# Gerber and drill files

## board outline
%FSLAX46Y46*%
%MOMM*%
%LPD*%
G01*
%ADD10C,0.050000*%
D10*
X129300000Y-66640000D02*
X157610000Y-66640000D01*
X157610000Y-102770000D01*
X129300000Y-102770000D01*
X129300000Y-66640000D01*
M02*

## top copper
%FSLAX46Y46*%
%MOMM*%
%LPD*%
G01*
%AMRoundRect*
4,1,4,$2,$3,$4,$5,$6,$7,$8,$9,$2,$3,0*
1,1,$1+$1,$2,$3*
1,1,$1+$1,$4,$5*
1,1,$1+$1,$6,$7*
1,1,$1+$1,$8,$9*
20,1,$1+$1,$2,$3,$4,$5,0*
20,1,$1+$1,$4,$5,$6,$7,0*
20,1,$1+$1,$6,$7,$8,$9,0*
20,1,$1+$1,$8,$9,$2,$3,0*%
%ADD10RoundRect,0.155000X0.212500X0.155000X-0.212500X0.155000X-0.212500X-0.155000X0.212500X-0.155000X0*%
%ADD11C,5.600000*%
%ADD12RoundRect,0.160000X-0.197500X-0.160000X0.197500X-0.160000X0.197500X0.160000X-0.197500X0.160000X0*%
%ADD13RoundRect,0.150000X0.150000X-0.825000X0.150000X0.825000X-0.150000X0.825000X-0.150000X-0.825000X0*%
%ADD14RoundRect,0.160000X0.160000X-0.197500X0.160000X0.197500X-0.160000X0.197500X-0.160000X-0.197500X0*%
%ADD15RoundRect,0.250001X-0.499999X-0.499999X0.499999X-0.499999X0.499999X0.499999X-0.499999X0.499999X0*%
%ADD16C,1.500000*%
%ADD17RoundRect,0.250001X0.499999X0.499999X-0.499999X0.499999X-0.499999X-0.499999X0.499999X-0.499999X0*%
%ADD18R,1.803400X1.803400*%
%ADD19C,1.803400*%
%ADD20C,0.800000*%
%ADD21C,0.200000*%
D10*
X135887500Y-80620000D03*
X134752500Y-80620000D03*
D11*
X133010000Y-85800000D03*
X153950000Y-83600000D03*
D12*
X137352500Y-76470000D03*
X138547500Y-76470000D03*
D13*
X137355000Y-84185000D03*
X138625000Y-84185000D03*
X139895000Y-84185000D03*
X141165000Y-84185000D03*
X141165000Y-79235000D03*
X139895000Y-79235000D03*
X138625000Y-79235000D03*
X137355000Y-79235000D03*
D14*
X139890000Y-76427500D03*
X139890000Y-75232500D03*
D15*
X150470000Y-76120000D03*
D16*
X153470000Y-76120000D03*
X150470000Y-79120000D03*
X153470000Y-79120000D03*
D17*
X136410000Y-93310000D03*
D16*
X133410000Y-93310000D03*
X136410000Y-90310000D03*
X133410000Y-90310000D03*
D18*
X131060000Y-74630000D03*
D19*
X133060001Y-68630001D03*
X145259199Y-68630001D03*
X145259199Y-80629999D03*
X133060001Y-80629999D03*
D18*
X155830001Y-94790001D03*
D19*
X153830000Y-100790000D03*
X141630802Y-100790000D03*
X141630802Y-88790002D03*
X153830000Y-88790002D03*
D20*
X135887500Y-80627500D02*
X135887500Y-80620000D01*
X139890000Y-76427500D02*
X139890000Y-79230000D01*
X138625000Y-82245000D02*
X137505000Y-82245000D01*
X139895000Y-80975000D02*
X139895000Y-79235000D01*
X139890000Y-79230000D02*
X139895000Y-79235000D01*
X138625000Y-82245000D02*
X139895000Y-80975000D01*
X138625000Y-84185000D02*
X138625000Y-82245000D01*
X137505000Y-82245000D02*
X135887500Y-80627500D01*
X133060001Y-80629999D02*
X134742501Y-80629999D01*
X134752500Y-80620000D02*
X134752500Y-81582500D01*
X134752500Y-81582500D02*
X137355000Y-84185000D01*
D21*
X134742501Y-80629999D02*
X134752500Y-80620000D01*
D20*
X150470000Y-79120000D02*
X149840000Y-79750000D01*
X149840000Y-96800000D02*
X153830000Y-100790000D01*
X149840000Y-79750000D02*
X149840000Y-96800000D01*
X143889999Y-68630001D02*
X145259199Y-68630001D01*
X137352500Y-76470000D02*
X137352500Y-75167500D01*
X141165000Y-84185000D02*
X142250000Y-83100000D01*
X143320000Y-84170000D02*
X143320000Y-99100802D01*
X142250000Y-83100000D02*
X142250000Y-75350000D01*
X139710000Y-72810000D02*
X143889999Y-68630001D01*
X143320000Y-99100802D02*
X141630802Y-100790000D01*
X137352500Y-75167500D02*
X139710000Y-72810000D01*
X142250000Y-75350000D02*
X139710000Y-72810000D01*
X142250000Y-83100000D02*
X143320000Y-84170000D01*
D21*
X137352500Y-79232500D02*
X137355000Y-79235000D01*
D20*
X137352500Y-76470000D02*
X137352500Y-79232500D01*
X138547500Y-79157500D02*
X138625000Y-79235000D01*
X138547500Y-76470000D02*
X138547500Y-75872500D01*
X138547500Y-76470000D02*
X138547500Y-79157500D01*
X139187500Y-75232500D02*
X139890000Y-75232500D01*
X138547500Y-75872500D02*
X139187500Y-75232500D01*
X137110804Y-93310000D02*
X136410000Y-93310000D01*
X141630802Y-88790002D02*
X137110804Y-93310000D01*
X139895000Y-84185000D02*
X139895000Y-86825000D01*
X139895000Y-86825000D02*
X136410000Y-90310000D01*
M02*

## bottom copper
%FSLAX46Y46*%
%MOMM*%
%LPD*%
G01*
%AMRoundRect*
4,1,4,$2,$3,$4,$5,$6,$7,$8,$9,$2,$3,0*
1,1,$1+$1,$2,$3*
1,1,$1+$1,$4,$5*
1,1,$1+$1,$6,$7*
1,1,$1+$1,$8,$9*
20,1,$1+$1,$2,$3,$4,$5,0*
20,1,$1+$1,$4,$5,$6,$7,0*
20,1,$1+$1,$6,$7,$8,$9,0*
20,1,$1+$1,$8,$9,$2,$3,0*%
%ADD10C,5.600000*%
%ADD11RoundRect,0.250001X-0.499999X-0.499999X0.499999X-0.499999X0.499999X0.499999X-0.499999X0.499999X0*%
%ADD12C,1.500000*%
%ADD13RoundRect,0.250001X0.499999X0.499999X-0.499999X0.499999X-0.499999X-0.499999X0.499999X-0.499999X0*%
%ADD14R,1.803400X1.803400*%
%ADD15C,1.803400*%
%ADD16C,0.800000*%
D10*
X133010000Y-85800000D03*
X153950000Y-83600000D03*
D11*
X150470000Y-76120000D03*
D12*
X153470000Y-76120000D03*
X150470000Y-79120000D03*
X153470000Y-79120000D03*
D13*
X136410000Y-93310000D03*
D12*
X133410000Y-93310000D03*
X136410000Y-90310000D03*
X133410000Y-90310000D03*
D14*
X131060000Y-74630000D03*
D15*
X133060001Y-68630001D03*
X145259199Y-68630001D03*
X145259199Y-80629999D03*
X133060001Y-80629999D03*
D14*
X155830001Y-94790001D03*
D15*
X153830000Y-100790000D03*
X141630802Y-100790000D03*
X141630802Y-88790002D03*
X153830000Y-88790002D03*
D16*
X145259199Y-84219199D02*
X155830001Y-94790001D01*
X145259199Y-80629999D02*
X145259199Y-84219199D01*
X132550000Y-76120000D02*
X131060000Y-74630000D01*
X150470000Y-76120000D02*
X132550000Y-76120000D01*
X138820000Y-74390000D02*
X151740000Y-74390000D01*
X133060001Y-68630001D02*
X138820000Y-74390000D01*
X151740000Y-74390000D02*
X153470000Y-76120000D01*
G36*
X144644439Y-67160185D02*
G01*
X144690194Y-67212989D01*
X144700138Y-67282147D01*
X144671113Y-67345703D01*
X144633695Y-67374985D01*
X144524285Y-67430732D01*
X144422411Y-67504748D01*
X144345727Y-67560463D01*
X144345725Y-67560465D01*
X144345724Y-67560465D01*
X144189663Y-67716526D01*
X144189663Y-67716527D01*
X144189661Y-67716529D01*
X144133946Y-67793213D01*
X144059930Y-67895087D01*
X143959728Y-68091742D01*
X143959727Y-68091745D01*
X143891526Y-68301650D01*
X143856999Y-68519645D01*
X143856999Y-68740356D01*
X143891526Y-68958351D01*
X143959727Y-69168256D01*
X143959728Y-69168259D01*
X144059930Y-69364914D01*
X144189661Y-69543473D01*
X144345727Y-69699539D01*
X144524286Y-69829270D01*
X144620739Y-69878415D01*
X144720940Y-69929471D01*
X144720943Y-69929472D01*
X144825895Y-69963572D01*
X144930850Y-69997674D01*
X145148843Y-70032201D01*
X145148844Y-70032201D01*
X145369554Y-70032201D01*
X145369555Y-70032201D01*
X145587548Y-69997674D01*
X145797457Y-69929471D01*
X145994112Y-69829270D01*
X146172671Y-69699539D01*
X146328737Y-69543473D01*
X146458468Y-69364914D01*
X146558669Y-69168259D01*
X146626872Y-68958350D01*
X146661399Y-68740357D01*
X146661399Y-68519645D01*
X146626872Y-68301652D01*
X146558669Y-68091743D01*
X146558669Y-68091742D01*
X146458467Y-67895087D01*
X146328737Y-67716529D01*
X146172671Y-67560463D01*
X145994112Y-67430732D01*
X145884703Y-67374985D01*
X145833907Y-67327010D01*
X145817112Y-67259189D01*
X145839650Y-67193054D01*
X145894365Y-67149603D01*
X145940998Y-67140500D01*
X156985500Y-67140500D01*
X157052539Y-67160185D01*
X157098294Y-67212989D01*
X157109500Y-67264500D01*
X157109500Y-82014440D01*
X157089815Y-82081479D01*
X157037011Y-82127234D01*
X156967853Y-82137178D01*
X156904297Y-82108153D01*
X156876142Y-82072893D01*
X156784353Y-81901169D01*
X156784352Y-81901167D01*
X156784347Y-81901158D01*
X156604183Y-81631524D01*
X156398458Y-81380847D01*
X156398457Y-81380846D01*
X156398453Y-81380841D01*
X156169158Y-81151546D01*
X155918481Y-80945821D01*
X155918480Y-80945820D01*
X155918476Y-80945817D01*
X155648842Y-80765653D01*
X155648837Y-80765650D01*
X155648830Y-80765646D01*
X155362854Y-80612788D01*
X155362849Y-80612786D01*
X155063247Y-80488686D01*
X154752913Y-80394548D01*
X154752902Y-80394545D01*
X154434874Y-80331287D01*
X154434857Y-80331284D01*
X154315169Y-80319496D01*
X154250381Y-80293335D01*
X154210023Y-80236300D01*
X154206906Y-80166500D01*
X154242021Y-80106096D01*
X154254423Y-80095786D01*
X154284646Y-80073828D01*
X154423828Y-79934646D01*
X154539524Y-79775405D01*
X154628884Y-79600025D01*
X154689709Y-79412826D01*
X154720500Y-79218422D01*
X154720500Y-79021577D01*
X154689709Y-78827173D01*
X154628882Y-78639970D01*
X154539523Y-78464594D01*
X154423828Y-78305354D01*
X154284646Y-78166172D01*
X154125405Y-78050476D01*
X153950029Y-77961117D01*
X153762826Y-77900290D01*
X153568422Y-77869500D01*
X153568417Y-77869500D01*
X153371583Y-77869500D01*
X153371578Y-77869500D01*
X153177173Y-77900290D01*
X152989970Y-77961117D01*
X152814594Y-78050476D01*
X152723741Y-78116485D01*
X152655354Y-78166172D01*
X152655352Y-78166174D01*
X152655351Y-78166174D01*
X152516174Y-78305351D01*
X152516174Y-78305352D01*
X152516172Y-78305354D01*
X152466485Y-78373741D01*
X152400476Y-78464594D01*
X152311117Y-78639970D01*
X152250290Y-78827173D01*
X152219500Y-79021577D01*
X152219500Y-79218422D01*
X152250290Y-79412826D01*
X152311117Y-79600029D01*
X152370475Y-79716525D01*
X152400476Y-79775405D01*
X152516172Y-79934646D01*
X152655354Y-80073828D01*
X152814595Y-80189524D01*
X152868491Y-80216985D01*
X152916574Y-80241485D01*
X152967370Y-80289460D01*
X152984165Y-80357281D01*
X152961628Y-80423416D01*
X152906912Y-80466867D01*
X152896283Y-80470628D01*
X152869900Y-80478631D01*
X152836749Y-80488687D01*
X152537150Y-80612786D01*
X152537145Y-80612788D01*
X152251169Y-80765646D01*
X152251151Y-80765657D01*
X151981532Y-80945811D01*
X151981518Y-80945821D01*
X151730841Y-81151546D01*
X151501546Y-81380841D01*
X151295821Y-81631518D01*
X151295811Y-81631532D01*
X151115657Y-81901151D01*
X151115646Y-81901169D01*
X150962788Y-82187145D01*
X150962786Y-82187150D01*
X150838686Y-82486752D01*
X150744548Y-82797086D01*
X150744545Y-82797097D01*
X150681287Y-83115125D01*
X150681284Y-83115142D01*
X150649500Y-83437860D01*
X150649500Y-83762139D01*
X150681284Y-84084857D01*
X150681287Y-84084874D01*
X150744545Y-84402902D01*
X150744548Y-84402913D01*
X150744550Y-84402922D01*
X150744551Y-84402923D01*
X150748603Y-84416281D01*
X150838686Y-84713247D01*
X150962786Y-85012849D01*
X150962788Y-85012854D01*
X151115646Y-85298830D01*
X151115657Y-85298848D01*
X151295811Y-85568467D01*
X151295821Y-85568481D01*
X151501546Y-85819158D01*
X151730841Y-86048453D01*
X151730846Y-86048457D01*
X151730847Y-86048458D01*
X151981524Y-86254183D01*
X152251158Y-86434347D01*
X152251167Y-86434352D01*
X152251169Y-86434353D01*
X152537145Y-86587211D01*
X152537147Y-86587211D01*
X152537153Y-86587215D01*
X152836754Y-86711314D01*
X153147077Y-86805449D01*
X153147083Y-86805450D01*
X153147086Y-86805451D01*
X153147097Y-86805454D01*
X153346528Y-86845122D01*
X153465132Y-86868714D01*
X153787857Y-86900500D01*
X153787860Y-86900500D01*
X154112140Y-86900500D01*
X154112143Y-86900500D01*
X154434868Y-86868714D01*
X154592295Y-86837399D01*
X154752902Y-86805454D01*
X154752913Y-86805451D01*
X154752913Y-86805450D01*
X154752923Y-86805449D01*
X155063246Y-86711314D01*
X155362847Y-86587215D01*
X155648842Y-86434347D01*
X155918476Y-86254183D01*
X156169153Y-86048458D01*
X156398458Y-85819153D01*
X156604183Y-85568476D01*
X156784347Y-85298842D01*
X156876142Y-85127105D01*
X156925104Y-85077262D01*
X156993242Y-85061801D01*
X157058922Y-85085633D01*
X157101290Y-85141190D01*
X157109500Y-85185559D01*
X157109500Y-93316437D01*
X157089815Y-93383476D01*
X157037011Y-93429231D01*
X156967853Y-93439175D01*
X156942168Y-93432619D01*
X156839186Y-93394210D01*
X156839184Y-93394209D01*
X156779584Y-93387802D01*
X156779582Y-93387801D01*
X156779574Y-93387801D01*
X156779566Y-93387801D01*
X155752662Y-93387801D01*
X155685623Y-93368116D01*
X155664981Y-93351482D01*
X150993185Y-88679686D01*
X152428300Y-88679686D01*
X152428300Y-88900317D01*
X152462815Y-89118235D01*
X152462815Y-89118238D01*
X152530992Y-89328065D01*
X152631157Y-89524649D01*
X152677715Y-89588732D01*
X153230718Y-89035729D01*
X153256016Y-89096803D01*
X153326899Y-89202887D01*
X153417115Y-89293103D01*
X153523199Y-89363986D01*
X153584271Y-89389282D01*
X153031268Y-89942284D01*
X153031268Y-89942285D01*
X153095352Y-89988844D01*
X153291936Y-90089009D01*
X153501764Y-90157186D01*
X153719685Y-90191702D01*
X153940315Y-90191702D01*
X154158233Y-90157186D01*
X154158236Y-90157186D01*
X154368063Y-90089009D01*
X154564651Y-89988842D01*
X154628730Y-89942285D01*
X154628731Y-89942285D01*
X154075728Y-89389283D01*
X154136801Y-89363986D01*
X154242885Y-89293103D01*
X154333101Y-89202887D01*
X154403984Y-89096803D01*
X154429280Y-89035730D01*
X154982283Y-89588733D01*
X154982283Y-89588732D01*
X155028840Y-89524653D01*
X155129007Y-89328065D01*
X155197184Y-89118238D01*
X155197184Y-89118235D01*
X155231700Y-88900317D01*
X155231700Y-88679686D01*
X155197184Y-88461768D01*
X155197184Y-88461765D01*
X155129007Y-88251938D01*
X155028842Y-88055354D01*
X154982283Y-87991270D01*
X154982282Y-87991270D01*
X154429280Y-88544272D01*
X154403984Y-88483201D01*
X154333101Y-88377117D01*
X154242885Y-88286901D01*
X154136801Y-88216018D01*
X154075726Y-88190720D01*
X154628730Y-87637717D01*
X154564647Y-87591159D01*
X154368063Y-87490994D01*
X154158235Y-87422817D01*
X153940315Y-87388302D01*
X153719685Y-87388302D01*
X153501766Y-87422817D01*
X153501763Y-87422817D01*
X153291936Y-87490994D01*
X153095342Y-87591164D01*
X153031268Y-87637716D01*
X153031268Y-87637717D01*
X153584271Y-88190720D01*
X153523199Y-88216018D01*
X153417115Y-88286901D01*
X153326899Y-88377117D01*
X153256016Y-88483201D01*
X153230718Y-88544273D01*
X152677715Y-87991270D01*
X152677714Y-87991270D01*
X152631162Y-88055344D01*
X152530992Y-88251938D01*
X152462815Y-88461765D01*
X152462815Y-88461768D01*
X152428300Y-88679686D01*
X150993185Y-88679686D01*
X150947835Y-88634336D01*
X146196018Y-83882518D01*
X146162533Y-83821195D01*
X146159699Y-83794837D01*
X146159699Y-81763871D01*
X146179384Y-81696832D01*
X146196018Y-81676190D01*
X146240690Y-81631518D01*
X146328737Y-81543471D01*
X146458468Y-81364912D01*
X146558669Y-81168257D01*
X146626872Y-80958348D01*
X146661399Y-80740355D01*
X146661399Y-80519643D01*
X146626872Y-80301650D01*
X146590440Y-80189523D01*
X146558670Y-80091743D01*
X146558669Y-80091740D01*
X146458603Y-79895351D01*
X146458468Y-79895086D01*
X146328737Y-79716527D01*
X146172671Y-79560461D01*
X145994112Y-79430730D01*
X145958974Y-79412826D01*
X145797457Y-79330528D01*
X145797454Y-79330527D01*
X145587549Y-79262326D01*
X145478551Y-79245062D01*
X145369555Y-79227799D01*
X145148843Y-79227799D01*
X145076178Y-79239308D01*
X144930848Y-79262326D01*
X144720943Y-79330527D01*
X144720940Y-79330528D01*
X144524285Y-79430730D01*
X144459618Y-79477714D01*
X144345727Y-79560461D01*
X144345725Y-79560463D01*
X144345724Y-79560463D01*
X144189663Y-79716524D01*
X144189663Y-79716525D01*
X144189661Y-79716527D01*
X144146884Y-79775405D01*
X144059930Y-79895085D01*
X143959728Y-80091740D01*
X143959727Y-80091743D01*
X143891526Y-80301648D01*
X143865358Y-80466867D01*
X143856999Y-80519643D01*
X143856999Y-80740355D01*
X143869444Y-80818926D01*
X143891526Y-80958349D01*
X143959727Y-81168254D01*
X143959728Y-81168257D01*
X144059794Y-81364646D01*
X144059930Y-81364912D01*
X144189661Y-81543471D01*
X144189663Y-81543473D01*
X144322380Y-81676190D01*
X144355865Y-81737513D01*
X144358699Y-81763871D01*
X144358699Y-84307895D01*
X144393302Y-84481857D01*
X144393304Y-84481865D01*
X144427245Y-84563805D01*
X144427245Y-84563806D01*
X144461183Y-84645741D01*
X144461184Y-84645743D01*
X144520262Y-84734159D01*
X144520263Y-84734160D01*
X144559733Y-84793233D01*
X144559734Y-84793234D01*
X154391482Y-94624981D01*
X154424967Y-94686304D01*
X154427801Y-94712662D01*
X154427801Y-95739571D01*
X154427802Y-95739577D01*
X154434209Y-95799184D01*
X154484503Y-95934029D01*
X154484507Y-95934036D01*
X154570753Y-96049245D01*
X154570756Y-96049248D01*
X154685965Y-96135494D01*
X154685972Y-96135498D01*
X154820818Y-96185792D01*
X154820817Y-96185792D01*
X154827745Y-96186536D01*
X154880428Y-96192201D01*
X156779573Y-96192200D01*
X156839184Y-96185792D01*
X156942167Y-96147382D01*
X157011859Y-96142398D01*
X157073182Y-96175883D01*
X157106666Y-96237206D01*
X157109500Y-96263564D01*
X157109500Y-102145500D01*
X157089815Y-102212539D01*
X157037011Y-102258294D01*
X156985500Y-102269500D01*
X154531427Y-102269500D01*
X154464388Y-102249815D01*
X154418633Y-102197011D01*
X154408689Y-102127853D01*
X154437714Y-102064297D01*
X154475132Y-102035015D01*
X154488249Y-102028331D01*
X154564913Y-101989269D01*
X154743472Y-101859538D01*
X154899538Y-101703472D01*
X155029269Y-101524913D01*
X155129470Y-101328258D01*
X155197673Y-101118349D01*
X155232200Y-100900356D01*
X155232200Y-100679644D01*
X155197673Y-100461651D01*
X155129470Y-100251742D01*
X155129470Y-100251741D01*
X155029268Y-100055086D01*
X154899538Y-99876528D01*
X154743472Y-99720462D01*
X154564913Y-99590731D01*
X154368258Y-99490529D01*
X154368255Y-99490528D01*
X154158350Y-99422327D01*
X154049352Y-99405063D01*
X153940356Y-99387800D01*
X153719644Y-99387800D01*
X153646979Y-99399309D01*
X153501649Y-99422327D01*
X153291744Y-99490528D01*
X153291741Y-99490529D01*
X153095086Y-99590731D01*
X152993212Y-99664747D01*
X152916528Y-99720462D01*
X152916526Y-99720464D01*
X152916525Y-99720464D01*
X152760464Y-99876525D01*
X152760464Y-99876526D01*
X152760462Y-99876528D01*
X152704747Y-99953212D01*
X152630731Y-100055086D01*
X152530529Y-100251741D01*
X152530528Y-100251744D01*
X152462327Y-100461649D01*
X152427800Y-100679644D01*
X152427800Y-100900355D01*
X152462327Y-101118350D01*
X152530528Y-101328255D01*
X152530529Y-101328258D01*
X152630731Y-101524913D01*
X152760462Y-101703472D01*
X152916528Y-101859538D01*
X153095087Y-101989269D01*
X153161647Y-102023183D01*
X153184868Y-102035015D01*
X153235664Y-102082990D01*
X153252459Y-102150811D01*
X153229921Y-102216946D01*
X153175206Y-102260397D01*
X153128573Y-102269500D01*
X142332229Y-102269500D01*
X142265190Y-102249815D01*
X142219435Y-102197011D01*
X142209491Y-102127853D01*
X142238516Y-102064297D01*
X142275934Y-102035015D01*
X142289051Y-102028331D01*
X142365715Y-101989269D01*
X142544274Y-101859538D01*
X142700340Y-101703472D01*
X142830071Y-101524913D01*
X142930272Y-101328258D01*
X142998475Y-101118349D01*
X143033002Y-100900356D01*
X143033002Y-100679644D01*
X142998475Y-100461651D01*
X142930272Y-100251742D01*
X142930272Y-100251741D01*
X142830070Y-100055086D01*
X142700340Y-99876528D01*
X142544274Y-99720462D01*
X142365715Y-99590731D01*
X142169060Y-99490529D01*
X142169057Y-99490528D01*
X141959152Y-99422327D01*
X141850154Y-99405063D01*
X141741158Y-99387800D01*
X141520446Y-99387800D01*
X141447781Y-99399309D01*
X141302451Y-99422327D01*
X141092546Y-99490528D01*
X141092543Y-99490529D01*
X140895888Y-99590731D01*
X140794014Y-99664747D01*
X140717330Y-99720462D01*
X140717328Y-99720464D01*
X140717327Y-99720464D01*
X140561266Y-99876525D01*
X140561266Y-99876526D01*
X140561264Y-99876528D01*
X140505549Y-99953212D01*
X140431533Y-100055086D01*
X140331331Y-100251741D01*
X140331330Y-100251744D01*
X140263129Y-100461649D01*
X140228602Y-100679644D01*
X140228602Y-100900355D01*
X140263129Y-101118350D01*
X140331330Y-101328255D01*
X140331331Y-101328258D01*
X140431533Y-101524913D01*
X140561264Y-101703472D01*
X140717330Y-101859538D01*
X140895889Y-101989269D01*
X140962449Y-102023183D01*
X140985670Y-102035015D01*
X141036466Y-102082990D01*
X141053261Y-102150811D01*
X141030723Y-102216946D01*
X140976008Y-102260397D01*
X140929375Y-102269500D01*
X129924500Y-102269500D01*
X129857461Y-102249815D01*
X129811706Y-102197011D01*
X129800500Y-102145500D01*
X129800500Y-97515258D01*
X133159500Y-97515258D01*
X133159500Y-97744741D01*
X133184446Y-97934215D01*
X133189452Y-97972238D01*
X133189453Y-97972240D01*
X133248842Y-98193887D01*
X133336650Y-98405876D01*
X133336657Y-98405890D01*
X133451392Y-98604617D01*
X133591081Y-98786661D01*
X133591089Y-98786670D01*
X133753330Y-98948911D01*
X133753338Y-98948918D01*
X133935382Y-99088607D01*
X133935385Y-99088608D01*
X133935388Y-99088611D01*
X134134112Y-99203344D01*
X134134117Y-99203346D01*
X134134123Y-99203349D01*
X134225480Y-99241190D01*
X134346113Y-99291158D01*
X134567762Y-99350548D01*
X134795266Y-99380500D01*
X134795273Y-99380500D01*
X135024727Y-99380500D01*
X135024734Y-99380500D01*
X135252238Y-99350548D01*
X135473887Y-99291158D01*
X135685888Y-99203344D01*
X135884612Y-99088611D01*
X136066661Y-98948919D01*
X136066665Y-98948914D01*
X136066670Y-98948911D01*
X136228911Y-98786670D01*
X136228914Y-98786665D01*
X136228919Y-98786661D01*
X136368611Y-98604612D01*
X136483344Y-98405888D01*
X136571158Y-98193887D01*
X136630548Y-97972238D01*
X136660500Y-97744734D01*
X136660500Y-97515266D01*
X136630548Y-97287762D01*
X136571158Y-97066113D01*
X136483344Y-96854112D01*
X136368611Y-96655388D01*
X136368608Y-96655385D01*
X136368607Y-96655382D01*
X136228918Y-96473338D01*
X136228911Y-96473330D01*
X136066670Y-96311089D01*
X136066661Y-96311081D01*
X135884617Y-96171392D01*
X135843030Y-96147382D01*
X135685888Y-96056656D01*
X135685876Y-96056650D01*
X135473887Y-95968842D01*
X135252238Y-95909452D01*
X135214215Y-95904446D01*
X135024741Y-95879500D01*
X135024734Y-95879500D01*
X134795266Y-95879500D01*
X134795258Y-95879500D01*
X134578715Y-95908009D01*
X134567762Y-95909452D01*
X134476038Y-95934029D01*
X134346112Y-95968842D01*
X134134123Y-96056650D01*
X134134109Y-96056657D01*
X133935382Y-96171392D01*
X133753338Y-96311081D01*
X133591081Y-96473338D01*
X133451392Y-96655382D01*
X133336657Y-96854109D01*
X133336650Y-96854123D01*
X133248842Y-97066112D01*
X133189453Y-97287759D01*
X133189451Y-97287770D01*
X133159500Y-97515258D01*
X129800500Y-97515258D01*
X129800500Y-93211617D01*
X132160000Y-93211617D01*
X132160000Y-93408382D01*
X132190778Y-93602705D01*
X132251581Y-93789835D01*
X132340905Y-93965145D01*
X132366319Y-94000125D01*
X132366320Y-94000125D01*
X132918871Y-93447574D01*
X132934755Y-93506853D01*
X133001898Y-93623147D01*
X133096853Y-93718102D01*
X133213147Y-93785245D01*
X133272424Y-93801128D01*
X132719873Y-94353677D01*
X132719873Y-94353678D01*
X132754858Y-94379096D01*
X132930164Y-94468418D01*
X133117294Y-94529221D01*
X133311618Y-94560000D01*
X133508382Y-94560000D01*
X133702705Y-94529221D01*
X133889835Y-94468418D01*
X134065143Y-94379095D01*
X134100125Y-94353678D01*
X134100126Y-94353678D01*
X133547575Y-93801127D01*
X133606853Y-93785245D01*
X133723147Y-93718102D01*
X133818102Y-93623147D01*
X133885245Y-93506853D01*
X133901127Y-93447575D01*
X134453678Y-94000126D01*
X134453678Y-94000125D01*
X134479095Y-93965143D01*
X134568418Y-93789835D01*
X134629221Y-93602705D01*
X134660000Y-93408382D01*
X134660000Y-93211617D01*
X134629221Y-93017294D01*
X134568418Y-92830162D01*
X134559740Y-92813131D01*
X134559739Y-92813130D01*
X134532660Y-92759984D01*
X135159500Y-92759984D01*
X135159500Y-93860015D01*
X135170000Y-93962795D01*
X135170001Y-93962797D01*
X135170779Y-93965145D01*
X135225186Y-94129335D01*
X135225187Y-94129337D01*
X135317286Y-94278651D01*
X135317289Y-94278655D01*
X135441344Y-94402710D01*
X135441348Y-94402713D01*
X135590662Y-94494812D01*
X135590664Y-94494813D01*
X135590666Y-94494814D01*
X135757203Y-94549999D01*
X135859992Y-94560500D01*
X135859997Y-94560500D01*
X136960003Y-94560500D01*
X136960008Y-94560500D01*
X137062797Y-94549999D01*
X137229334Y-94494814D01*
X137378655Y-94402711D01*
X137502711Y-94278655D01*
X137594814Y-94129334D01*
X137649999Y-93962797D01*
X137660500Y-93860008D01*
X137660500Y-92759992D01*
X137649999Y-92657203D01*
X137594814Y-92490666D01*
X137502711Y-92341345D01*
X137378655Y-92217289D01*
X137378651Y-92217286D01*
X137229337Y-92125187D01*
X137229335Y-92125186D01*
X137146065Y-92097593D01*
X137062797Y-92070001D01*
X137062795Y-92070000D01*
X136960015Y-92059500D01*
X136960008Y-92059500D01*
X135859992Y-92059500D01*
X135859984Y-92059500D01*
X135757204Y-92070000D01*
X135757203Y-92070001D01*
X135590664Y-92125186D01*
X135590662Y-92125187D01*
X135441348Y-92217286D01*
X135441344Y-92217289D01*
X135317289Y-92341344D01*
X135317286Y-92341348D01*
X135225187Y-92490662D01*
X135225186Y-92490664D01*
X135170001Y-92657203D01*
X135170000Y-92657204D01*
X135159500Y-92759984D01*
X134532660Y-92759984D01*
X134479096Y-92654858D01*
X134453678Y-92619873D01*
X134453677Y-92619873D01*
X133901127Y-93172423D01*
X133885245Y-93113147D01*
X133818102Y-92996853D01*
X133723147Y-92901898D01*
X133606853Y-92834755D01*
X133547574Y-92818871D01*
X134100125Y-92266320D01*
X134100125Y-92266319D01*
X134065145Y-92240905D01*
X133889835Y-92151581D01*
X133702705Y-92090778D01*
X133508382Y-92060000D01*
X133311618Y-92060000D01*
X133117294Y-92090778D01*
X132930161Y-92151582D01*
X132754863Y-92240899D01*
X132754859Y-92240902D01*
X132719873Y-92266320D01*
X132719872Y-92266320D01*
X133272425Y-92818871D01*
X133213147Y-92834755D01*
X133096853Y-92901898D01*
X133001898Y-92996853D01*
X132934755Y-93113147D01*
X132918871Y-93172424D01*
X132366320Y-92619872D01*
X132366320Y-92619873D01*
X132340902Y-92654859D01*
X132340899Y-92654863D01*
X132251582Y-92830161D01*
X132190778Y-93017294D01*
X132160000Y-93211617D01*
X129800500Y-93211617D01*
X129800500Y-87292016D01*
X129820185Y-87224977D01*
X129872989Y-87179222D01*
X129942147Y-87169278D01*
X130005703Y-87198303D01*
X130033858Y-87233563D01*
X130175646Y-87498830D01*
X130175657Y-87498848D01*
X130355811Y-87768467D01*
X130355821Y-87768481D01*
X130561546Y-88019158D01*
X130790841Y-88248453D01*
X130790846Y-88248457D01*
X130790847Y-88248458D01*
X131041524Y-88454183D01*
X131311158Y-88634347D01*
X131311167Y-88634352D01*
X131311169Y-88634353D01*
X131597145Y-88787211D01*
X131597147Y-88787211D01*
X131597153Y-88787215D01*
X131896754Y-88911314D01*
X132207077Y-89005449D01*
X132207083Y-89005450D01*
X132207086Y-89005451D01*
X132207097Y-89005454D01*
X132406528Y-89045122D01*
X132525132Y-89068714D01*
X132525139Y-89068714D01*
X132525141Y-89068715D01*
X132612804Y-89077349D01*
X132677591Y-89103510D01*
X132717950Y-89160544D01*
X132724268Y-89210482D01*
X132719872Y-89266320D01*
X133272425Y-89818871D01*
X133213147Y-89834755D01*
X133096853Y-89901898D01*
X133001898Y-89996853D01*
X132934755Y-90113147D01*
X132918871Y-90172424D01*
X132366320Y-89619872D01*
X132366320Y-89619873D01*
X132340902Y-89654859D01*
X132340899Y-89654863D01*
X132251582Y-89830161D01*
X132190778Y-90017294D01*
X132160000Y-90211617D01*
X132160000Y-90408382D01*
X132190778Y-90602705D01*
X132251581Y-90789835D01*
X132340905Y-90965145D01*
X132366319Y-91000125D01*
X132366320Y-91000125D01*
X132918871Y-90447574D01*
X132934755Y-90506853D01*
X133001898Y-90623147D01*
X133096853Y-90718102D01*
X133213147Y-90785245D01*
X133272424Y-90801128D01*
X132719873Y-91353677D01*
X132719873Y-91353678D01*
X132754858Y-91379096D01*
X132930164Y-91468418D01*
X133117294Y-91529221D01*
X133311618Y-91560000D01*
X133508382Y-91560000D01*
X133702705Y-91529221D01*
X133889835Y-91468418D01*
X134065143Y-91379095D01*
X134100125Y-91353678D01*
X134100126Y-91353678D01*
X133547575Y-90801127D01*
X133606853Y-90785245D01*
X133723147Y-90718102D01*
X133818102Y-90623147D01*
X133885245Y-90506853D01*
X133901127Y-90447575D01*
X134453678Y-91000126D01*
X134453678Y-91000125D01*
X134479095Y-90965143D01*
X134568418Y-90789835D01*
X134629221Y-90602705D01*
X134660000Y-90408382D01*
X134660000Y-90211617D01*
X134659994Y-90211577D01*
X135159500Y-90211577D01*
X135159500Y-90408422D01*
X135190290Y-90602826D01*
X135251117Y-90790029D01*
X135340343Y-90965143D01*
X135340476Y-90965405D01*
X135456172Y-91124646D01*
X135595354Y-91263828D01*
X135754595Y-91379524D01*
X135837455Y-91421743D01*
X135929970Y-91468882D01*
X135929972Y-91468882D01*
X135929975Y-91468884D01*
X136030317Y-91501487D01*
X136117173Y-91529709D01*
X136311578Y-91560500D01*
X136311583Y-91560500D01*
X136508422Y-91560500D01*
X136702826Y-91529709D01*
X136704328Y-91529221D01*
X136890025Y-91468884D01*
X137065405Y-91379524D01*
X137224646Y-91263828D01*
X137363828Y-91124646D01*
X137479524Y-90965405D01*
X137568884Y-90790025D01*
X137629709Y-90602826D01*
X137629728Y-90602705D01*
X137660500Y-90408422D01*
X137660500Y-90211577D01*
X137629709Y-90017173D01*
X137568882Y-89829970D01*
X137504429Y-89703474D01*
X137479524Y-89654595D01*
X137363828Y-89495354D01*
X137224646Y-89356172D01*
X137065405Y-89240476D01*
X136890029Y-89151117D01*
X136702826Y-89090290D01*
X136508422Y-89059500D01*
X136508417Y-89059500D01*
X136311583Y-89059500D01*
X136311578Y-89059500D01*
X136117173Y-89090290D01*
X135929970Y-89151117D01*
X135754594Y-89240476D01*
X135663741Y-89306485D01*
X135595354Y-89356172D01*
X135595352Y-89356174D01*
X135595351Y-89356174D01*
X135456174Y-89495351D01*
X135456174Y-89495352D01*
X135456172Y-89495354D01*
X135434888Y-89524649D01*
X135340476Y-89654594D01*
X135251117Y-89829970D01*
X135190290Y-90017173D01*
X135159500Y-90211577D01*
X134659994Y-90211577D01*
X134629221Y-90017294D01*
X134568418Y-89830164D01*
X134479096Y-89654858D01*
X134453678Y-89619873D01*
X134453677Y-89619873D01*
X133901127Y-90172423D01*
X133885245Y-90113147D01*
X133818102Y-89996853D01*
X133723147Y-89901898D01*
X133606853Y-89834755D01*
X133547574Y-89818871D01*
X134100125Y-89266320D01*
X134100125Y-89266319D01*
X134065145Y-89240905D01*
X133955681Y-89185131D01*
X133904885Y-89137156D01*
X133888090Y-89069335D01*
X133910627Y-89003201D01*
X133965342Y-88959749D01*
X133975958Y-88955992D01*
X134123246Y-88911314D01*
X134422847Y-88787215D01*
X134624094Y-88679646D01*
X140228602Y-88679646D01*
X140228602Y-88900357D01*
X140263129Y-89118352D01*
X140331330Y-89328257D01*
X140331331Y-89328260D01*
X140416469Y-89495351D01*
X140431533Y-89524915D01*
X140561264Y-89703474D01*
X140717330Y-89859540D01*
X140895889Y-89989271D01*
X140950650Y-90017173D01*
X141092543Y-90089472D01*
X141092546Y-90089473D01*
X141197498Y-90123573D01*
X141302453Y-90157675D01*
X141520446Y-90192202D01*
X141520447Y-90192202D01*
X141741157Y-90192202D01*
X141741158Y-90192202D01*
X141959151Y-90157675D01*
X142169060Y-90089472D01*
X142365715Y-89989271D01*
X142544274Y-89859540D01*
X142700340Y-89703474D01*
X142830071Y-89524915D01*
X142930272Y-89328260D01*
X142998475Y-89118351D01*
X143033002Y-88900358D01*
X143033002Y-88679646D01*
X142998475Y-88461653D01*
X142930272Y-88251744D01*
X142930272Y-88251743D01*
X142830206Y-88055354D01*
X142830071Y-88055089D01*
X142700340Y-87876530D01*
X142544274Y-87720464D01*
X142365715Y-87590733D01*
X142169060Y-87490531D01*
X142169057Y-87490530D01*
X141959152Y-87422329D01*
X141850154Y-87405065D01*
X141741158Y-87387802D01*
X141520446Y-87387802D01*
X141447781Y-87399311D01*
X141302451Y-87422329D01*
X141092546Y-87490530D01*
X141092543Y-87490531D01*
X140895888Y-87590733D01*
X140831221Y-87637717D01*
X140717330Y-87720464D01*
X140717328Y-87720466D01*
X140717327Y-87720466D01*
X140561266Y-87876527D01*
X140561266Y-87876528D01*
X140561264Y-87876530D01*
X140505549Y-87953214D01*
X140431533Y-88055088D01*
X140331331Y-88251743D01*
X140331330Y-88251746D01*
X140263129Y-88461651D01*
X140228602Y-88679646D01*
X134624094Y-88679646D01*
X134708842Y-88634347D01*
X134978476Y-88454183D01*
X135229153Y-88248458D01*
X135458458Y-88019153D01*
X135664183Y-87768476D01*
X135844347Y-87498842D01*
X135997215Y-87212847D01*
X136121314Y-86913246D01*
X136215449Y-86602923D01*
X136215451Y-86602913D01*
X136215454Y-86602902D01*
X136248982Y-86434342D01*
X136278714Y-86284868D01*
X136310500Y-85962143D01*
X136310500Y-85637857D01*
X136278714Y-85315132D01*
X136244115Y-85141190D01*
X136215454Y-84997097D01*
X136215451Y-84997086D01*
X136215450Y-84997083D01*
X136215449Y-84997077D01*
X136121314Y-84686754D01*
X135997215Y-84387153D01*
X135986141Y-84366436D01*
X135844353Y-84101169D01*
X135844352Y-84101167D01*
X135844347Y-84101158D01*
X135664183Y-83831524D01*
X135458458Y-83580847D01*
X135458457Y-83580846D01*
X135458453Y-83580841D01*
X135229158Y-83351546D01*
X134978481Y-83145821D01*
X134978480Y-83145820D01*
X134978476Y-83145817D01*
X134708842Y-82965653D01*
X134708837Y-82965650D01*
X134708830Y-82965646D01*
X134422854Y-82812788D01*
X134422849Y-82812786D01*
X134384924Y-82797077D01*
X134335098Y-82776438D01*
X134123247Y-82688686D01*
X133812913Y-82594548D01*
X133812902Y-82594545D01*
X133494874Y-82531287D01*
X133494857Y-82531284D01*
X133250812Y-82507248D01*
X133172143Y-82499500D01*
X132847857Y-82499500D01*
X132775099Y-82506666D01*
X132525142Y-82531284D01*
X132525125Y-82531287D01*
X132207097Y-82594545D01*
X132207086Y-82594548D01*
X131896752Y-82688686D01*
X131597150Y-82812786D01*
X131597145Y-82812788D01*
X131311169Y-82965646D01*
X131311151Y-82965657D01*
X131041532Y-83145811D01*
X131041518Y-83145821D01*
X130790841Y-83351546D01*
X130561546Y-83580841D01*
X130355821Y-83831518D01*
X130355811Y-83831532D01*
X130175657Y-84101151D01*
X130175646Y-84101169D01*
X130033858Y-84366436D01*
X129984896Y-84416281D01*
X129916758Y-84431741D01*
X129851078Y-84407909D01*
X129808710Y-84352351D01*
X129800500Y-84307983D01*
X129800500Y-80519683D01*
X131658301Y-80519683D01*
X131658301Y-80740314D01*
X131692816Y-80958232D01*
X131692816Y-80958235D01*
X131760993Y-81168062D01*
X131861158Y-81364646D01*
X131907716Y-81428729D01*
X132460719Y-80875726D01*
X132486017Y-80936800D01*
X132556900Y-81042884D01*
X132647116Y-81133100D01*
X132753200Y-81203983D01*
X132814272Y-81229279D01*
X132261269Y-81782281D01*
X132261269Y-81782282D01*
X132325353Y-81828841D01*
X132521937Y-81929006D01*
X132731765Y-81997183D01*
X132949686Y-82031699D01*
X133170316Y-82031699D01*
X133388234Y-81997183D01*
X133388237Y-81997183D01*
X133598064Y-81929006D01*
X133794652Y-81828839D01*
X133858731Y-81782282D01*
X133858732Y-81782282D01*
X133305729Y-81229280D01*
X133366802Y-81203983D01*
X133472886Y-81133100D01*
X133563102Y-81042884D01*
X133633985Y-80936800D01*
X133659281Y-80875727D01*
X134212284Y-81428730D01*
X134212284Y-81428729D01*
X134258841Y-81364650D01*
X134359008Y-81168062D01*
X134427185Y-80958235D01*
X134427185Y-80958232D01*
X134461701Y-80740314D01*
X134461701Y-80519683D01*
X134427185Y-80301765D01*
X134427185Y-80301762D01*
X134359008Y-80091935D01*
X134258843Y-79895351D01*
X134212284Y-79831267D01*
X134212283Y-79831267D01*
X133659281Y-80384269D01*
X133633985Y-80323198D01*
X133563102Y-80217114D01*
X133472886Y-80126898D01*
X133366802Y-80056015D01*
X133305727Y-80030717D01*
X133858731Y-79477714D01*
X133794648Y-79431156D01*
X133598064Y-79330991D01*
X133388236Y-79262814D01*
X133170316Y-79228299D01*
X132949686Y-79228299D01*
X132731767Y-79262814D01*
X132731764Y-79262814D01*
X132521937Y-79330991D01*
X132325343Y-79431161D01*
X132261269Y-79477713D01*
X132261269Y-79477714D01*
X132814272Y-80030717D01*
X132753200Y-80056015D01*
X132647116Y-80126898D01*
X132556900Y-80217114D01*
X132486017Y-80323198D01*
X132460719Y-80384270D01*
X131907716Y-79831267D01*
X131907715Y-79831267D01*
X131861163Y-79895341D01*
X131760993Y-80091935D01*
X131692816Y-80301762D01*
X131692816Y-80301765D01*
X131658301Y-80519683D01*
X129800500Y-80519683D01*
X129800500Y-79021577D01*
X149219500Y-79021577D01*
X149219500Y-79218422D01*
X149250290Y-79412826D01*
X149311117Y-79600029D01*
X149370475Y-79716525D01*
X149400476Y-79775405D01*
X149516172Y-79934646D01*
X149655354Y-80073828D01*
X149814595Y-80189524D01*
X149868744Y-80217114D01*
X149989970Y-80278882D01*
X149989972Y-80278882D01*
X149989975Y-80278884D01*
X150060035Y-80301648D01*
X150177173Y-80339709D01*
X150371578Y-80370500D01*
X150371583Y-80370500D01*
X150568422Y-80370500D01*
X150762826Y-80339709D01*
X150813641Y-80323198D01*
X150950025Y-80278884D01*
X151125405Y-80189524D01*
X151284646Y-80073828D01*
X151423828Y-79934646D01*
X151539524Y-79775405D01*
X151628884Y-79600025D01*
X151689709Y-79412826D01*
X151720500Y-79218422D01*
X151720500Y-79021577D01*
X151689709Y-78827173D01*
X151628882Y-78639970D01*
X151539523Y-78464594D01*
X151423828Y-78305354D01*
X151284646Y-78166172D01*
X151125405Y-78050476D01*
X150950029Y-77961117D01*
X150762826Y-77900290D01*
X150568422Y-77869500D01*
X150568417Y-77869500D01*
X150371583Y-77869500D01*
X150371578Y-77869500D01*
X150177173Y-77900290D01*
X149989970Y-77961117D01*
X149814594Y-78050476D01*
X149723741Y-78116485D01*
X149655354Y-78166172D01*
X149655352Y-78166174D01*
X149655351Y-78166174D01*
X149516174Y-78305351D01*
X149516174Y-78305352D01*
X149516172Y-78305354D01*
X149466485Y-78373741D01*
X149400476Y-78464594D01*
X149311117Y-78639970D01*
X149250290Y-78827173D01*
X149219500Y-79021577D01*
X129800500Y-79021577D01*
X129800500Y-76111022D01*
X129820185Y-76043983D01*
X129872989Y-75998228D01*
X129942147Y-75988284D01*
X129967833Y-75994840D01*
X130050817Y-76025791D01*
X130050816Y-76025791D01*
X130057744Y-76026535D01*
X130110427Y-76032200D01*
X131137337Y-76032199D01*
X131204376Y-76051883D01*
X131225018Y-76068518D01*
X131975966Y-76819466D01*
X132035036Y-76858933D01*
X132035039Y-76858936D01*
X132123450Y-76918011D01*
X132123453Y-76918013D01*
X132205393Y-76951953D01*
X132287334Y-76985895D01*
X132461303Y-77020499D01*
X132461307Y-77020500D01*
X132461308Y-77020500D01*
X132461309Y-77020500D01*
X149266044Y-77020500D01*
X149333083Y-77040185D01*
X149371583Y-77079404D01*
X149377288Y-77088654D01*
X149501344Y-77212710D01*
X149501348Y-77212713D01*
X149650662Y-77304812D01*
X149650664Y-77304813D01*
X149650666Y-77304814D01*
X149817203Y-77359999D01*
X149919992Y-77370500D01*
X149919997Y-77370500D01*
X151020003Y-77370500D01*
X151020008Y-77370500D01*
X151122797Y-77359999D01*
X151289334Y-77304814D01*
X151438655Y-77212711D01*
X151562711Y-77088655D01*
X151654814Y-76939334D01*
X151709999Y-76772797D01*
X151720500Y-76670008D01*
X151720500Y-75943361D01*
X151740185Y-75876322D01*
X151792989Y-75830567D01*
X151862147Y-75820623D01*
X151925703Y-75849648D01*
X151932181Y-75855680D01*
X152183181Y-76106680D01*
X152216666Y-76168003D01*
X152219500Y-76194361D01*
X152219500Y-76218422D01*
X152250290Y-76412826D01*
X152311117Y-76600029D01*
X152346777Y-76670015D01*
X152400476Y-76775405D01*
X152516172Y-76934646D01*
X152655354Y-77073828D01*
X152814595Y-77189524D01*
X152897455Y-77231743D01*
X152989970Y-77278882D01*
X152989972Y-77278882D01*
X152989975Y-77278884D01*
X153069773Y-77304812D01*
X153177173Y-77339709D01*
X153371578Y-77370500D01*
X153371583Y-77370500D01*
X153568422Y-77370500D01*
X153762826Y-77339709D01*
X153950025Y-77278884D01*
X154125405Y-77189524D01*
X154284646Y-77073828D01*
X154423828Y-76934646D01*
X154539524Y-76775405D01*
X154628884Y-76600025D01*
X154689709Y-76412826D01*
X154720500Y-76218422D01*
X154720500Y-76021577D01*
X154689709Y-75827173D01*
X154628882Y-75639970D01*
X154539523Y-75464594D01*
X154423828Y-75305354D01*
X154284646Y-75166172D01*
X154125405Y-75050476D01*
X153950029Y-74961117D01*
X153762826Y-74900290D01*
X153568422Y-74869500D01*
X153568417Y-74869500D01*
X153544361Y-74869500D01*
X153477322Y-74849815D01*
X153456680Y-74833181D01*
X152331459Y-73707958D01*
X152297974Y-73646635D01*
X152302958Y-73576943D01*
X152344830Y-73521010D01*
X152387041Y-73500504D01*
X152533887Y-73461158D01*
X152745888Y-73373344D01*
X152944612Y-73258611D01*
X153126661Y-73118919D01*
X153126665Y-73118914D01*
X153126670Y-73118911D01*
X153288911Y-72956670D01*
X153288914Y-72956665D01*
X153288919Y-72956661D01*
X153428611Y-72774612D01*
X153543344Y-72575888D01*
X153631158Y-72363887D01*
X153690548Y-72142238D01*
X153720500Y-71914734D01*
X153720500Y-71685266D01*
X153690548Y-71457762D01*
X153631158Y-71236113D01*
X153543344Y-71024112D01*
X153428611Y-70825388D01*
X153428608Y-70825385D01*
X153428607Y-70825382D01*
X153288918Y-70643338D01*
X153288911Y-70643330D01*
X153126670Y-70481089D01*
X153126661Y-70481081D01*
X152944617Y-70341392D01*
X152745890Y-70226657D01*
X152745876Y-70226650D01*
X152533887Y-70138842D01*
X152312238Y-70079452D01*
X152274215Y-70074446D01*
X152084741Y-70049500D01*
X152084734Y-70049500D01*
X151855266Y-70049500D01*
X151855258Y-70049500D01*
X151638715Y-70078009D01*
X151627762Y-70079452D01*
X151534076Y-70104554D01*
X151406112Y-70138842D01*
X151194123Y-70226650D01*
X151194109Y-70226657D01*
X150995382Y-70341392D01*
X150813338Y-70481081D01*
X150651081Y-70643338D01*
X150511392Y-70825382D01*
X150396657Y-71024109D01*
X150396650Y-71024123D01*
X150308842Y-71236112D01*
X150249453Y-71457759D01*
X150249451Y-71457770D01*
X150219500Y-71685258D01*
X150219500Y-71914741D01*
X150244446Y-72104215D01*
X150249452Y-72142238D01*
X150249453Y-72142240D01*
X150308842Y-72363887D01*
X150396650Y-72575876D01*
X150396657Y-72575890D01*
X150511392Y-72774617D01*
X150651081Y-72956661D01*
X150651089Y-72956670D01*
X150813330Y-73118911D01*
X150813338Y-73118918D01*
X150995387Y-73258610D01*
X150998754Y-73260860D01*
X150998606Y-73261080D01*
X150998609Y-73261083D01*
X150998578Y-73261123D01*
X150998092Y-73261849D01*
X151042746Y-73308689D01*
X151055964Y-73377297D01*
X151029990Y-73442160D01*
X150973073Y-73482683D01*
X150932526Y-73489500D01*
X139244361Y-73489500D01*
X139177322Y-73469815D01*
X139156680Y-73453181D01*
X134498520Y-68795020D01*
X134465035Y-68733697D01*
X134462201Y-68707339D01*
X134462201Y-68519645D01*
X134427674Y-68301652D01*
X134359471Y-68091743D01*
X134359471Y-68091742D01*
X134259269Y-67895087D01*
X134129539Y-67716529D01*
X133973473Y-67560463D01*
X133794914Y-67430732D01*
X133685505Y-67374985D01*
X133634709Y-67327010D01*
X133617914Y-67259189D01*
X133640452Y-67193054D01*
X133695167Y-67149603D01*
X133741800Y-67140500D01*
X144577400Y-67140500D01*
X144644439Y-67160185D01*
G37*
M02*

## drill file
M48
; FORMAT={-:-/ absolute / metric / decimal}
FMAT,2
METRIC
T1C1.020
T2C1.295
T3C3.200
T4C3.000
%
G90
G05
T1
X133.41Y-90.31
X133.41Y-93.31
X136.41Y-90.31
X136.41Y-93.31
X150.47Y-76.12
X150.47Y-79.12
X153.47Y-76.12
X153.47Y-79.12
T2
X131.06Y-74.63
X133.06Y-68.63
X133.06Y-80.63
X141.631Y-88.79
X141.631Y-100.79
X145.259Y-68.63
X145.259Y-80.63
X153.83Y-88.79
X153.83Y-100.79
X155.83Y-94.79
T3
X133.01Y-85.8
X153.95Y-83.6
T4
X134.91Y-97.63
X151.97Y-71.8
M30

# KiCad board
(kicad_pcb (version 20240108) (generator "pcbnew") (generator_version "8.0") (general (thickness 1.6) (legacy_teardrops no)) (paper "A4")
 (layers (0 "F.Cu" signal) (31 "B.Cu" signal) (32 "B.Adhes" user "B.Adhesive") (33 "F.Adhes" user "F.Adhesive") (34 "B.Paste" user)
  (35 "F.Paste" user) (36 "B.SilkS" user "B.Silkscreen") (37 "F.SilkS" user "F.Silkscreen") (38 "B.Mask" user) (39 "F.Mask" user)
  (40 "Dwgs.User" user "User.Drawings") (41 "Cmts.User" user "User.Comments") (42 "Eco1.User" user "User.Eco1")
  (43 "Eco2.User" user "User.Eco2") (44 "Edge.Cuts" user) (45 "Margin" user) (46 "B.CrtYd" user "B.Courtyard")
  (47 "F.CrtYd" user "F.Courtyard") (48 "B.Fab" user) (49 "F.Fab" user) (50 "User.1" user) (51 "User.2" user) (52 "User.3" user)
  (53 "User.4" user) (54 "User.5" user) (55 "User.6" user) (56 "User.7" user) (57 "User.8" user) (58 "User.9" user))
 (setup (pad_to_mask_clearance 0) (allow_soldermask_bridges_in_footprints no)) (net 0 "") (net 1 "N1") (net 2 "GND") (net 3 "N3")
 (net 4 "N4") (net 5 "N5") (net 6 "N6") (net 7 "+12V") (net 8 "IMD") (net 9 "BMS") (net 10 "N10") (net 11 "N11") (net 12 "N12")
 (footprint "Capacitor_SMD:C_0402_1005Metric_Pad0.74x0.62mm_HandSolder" (layer "F.Cu") (at 135.32 80.62 180)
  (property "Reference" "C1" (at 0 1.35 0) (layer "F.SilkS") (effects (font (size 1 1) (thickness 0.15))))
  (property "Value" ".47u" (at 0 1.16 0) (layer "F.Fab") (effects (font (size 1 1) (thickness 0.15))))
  (pad "1" smd roundrect (at -0.5675 0 180) (size 0.735 0.62) (layers "F.Cu" "F.Paste" "F.Mask") (roundrect_rratio 0.25) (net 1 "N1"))
  (pad "2" smd roundrect (at 0.5675 0 180) (size 0.735 0.62) (layers "F.Cu" "F.Paste" "F.Mask") (roundrect_rratio 0.25) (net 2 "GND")))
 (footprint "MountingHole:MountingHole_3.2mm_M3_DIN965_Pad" (layer "F.Cu") (at 133.01 85.8)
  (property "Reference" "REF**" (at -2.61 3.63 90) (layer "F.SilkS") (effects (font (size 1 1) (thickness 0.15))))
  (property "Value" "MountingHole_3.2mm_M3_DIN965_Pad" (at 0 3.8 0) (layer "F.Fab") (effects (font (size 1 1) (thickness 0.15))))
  (pad "1" thru_hole circle (at 0 0) (size 5.6 5.6) (drill 3.2) (layers "*.Cu" "*.Mask") (remove_unused_layers no)))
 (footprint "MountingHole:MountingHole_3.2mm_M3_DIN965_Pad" (layer "F.Cu") (at 153.95 83.6)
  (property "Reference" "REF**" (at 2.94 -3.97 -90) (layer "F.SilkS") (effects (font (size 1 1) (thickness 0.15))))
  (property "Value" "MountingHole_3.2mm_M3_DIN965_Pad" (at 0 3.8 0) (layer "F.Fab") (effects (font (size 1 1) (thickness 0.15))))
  (pad "1" thru_hole circle (at 0 0) (size 5.6 5.6) (drill 3.2) (layers "*.Cu" "*.Mask") (remove_unused_layers no)))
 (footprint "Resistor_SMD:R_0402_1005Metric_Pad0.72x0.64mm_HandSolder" (layer "F.Cu") (at 137.95 76.47)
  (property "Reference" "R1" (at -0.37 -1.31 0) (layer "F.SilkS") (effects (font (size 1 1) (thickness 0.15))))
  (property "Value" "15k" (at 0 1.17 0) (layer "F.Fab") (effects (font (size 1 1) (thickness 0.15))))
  (pad "1" smd roundrect (at -0.5975 0) (size 0.715 0.64) (layers "F.Cu" "F.Paste" "F.Mask") (roundrect_rratio 0.25) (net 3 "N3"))
  (pad "2" smd roundrect (at 0.5975 0) (size 0.715 0.64) (layers "F.Cu" "F.Paste" "F.Mask") (roundrect_rratio 0.25) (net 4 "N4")))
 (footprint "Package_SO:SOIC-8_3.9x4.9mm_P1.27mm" (layer "F.Cu") (at 139.26 81.71 90)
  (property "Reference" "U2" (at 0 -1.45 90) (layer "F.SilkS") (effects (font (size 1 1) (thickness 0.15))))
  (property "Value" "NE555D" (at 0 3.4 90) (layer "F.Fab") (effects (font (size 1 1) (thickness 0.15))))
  (pad "1" smd roundrect (at -2.475 -1.905 90) (size 1.95 0.6) (layers "F.Cu" "F.Paste" "F.Mask") (roundrect_rratio 0.25) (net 2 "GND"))
  (pad "2" smd roundrect (at -2.475 -0.635 90) (size 1.95 0.6) (layers "F.Cu" "F.Paste" "F.Mask") (roundrect_rratio 0.25) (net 1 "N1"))
  (pad "3" smd roundrect (at -2.475 0.635 90) (size 1.95 0.6) (layers "F.Cu" "F.Paste" "F.Mask") (roundrect_rratio 0.25) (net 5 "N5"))
  (pad "4" smd roundrect (at -2.475 1.905 90) (size 1.95 0.6) (layers "F.Cu" "F.Paste" "F.Mask") (roundrect_rratio 0.25) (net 3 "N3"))
  (pad "5" smd roundrect (at 2.475 1.905 90) (size 1.95 0.6) (layers "F.Cu" "F.Paste" "F.Mask") (roundrect_rratio 0.25) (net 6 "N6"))
  (pad "6" smd roundrect (at 2.475 0.635 90) (size 1.95 0.6) (layers "F.Cu" "F.Paste" "F.Mask") (roundrect_rratio 0.25) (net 1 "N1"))
  (pad "7" smd roundrect (at 2.475 -0.635 90) (size 1.95 0.6) (layers "F.Cu" "F.Paste" "F.Mask") (roundrect_rratio 0.25) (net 4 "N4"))
  (pad "8" smd roundrect (at 2.475 -1.905 90) (size 1.95 0.6) (layers "F.Cu" "F.Paste" "F.Mask") (roundrect_rratio 0.25) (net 3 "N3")))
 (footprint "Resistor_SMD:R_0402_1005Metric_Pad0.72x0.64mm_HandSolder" (layer "F.Cu") (at 139.89 75.83 90)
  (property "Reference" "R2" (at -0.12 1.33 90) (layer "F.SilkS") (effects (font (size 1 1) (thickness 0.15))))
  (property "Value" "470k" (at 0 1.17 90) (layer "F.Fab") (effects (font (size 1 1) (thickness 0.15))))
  (pad "1" smd roundrect (at -0.5975 0 90) (size 0.715 0.64) (layers "F.Cu" "F.Paste" "F.Mask") (roundrect_rratio 0.25) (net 1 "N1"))
  (pad "2" smd roundrect (at 0.5975 0 90) (size 0.715 0.64) (layers "F.Cu" "F.Paste" "F.Mask") (roundrect_rratio 0.25) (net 4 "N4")))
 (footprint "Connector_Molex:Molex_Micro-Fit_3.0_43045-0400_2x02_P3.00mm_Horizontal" (layer "F.Cu") (at 150.47 76.12)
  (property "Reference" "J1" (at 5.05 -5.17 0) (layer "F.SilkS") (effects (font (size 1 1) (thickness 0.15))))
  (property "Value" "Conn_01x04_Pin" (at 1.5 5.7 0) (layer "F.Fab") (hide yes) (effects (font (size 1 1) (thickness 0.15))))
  (pad "" np_thru_hole circle (at 1.5 -4.32) (size 3 3) (drill 3) (layers "*.Cu" "*.Mask"))
  (pad "1" thru_hole roundrect (at 0 0) (size 1.5 1.5) (drill 1.02) (layers "*.Cu" "*.Mask") (remove_unused_layers no)
   (roundrect_rratio 0.166667) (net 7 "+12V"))
  (pad "2" thru_hole circle (at 3 0) (size 1.5 1.5) (drill 1.02) (layers "*.Cu" "*.Mask") (remove_unused_layers no) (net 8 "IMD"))
  (pad "3" thru_hole circle (at 0 3) (size 1.5 1.5) (drill 1.02) (layers "*.Cu" "*.Mask") (remove_unused_layers no) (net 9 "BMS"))
  (pad "4" thru_hole circle (at 3 3) (size 1.5 1.5) (drill 1.02) (layers "*.Cu" "*.Mask") (remove_unused_layers no) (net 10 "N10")))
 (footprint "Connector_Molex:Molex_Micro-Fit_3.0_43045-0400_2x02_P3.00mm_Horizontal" (layer "F.Cu") (at 136.41 93.31 180)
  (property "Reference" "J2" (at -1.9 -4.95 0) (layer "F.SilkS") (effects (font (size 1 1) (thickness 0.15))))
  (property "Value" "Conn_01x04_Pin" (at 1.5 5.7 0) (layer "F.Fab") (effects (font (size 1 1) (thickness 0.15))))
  (pad "" np_thru_hole circle (at 1.5 -4.32 180) (size 3 3) (drill 3) (layers "*.Cu" "*.Mask"))
  (pad "1" thru_hole roundrect (at 0 0 180) (size 1.5 1.5) (drill 1.02) (layers "*.Cu" "*.Mask") (remove_unused_layers no)
   (roundrect_rratio 0.166667) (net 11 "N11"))
  (pad "2" thru_hole circle (at 3 0 180) (size 1.5 1.5) (drill 1.02) (layers "*.Cu" "*.Mask") (remove_unused_layers no) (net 2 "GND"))
  (pad "3" thru_hole circle (at 0 3 180) (size 1.5 1.5) (drill 1.02) (layers "*.Cu" "*.Mask") (remove_unused_layers no) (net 5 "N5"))
  (pad "4" thru_hole circle (at 3 3 180) (size 1.5 1.5) (drill 1.02) (layers "*.Cu" "*.Mask") (remove_unused_layers no) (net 2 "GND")))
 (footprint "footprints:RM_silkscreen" (layer "B.Cu") (at 143.81 84.77 180)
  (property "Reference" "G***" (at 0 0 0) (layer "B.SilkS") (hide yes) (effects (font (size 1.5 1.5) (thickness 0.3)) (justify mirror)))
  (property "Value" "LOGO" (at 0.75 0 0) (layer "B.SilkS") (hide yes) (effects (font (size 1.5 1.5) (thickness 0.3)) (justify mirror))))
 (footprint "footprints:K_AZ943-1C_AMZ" (layer "B.Cu") (at 131.06 74.63 -90)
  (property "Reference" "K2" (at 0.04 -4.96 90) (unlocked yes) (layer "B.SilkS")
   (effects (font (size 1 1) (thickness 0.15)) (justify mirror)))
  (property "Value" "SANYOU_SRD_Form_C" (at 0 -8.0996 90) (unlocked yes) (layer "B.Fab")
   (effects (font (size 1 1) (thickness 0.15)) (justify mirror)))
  (pad "1" thru_hole rect (at 0 0 270) (size 1.8034 1.8034) (drill 1.2954) (layers "*.Cu" "*.Mask") (remove_unused_layers no) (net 7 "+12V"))
  (pad "2" thru_hole circle (at -5.999999 -2.000001 270) (size 1.8034 1.8034) (drill 1.2954) (layers "*.Cu" "*.Mask")
   (remove_unused_layers no) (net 8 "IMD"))
  (pad "3" thru_hole circle (at -5.999999 -14.199199 270) (size 1.8034 1.8034) (drill 1.2954) (layers "*.Cu" "*.Mask")
   (remove_unused_layers no) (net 3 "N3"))
  (pad "4" thru_hole circle (at 5.999999 -14.199199 270) (size 1.8034 1.8034) (drill 1.2954) (layers "*.Cu" "*.Mask")
   (remove_unused_layers no) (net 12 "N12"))
  (pad "5" thru_hole circle (at 5.999999 -2.000001 270) (size 1.8034 1.8034) (drill 1.2954) (layers "*.Cu" "*.Mask")
   (remove_unused_layers no) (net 2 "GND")))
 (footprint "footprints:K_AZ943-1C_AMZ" (layer "B.Cu") (at 155.830001 94.790001 90)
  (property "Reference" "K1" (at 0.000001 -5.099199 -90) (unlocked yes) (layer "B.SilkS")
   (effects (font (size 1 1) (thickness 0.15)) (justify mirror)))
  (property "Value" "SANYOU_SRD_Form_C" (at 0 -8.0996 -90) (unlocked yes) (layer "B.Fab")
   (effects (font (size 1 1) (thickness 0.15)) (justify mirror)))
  (pad "1" thru_hole rect (at 0 0 90) (size 1.8034 1.8034) (drill 1.2954) (layers "*.Cu" "*.Mask") (remove_unused_layers no) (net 12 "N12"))
  (pad "2" thru_hole circle (at -5.999999 -2.000001 90) (size 1.8034 1.8034) (drill 1.2954) (layers "*.Cu" "*.Mask")
   (remove_unused_layers no) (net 9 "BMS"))
  (pad "3" thru_hole circle (at -5.999999 -14.199199 90) (size 1.8034 1.8034) (drill 1.2954) (layers "*.Cu" "*.Mask")
   (remove_unused_layers no) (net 3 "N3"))
  (pad "4" thru_hole circle (at 5.999999 -14.199199 90) (size 1.8034 1.8034) (drill 1.2954) (layers "*.Cu" "*.Mask")
   (remove_unused_layers no) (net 11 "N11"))
  (pad "5" thru_hole circle (at 5.999999 -2.000001 90) (size 1.8034 1.8034) (drill 1.2954) (layers "*.Cu" "*.Mask")
   (remove_unused_layers no) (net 2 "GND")))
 (gr_rect (start 129.3 66.64) (end 157.61 102.77) (stroke (width 0.05) (type default)) (fill none) (layer "Edge.Cuts"))
 (segment (start 135.8875 80.6275) (end 135.8875 80.62) (width 0.8) (layer "F.Cu") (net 1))
 (segment (start 139.89 76.4275) (end 139.89 79.23) (width 0.8) (layer "F.Cu") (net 1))
 (segment (start 138.625 82.245) (end 137.505 82.245) (width 0.8) (layer "F.Cu") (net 1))
 (segment (start 139.895 80.975) (end 139.895 79.235) (width 0.8) (layer "F.Cu") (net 1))
 (segment (start 139.89 79.23) (end 139.895 79.235) (width 0.8) (layer "F.Cu") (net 1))
 (segment (start 138.625 82.245) (end 139.895 80.975) (width 0.8) (layer "F.Cu") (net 1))
 (segment (start 138.625 84.185) (end 138.625 82.245) (width 0.8) (layer "F.Cu") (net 1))
 (segment (start 137.505 82.245) (end 135.8875 80.6275) (width 0.8) (layer "F.Cu") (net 1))
 (segment (start 133.060001 80.629999) (end 134.742501 80.629999) (width 0.8) (layer "F.Cu") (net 2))
 (segment (start 134.7525 80.62) (end 134.7525 81.5825) (width 0.8) (layer "F.Cu") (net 2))
 (segment (start 134.7525 81.5825) (end 137.355 84.185) (width 0.8) (layer "F.Cu") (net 2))
 (segment (start 134.742501 80.629999) (end 134.7525 80.62) (width 0.2) (layer "F.Cu") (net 2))
 (segment (start 150.47 79.12) (end 149.84 79.75) (width 0.8) (layer "F.Cu") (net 9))
 (segment (start 149.84 96.8) (end 153.83 100.79) (width 0.8) (layer "F.Cu") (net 9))
 (segment (start 149.84 79.75) (end 149.84 96.8) (width 0.8) (layer "F.Cu") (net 9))
 (segment (start 145.259199 84.219199) (end 155.830001 94.790001) (width 0.8) (layer "B.Cu") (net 12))
 (segment (start 145.259199 80.629999) (end 145.259199 84.219199) (width 0.8) (layer "B.Cu") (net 12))
 (segment (start 143.889999 68.630001) (end 145.259199 68.630001) (width 0.8) (layer "F.Cu") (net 3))
 (segment (start 137.3525 76.47) (end 137.3525 75.1675) (width 0.8) (layer "F.Cu") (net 3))
 (segment (start 141.165 84.185) (end 142.25 83.1) (width 0.8) (layer "F.Cu") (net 3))
 (segment (start 143.32 84.17) (end 143.32 99.100802) (width 0.8) (layer "F.Cu") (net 3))
 (segment (start 142.25 83.1) (end 142.25 75.35) (width 0.8) (layer "F.Cu") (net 3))
 (segment (start 139.71 72.81) (end 143.889999 68.630001) (width 0.8) (layer "F.Cu") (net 3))
 (segment (start 143.32 99.100802) (end 141.630802 100.79) (width 0.8) (layer "F.Cu") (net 3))
 (segment (start 137.3525 75.1675) (end 139.71 72.81) (width 0.8) (layer "F.Cu") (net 3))
 (segment (start 142.25 75.35) (end 139.71 72.81) (width 0.8) (layer "F.Cu") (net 3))
 (segment (start 142.25 83.1) (end 143.32 84.17) (width 0.8) (layer "F.Cu") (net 3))
 (segment (start 137.3525 79.2325) (end 137.355 79.235) (width 0.2) (layer "F.Cu") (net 3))
 (segment (start 137.3525 76.47) (end 137.3525 79.2325) (width 0.8) (layer "F.Cu") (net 3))
 (segment (start 132.55 76.12) (end 131.06 74.63) (width 0.8) (layer "B.Cu") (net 7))
 (segment (start 150.47 76.12) (end 132.55 76.12) (width 0.8) (layer "B.Cu") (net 7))
 (segment (start 138.82 74.39) (end 151.74 74.39) (width 0.8) (layer "B.Cu") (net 8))
 (segment (start 133.060001 68.630001) (end 138.82 74.39) (width 0.8) (layer "B.Cu") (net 8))
 (segment (start 151.74 74.39) (end 153.47 76.12) (width 0.8) (layer "B.Cu") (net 8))
 (segment (start 138.5475 79.1575) (end 138.625 79.235) (width 0.8) (layer "F.Cu") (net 4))
 (segment (start 138.5475 76.47) (end 138.5475 75.8725) (width 0.8) (layer "F.Cu") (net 4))
 (segment (start 138.5475 76.47) (end 138.5475 79.1575) (width 0.8) (layer "F.Cu") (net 4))
 (segment (start 139.1875 75.2325) (end 139.89 75.2325) (width 0.8) (layer "F.Cu") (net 4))
 (segment (start 138.5475 75.8725) (end 139.1875 75.2325) (width 0.8) (layer "F.Cu") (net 4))
 (segment (start 137.110804 93.31) (end 136.41 93.31) (width 0.8) (layer "F.Cu") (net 11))
 (segment (start 141.630802 88.790002) (end 137.110804 93.31) (width 0.8) (layer "F.Cu") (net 11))
 (segment (start 139.895 84.185) (end 139.895 86.825) (width 0.8) (layer "F.Cu") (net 5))
 (segment (start 139.895 86.825) (end 136.41 90.31) (width 0.8) (layer "F.Cu") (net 5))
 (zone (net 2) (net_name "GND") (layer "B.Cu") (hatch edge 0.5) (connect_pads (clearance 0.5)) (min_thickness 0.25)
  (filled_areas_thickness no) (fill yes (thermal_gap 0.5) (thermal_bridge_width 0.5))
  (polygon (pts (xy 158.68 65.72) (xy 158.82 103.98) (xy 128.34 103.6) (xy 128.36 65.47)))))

